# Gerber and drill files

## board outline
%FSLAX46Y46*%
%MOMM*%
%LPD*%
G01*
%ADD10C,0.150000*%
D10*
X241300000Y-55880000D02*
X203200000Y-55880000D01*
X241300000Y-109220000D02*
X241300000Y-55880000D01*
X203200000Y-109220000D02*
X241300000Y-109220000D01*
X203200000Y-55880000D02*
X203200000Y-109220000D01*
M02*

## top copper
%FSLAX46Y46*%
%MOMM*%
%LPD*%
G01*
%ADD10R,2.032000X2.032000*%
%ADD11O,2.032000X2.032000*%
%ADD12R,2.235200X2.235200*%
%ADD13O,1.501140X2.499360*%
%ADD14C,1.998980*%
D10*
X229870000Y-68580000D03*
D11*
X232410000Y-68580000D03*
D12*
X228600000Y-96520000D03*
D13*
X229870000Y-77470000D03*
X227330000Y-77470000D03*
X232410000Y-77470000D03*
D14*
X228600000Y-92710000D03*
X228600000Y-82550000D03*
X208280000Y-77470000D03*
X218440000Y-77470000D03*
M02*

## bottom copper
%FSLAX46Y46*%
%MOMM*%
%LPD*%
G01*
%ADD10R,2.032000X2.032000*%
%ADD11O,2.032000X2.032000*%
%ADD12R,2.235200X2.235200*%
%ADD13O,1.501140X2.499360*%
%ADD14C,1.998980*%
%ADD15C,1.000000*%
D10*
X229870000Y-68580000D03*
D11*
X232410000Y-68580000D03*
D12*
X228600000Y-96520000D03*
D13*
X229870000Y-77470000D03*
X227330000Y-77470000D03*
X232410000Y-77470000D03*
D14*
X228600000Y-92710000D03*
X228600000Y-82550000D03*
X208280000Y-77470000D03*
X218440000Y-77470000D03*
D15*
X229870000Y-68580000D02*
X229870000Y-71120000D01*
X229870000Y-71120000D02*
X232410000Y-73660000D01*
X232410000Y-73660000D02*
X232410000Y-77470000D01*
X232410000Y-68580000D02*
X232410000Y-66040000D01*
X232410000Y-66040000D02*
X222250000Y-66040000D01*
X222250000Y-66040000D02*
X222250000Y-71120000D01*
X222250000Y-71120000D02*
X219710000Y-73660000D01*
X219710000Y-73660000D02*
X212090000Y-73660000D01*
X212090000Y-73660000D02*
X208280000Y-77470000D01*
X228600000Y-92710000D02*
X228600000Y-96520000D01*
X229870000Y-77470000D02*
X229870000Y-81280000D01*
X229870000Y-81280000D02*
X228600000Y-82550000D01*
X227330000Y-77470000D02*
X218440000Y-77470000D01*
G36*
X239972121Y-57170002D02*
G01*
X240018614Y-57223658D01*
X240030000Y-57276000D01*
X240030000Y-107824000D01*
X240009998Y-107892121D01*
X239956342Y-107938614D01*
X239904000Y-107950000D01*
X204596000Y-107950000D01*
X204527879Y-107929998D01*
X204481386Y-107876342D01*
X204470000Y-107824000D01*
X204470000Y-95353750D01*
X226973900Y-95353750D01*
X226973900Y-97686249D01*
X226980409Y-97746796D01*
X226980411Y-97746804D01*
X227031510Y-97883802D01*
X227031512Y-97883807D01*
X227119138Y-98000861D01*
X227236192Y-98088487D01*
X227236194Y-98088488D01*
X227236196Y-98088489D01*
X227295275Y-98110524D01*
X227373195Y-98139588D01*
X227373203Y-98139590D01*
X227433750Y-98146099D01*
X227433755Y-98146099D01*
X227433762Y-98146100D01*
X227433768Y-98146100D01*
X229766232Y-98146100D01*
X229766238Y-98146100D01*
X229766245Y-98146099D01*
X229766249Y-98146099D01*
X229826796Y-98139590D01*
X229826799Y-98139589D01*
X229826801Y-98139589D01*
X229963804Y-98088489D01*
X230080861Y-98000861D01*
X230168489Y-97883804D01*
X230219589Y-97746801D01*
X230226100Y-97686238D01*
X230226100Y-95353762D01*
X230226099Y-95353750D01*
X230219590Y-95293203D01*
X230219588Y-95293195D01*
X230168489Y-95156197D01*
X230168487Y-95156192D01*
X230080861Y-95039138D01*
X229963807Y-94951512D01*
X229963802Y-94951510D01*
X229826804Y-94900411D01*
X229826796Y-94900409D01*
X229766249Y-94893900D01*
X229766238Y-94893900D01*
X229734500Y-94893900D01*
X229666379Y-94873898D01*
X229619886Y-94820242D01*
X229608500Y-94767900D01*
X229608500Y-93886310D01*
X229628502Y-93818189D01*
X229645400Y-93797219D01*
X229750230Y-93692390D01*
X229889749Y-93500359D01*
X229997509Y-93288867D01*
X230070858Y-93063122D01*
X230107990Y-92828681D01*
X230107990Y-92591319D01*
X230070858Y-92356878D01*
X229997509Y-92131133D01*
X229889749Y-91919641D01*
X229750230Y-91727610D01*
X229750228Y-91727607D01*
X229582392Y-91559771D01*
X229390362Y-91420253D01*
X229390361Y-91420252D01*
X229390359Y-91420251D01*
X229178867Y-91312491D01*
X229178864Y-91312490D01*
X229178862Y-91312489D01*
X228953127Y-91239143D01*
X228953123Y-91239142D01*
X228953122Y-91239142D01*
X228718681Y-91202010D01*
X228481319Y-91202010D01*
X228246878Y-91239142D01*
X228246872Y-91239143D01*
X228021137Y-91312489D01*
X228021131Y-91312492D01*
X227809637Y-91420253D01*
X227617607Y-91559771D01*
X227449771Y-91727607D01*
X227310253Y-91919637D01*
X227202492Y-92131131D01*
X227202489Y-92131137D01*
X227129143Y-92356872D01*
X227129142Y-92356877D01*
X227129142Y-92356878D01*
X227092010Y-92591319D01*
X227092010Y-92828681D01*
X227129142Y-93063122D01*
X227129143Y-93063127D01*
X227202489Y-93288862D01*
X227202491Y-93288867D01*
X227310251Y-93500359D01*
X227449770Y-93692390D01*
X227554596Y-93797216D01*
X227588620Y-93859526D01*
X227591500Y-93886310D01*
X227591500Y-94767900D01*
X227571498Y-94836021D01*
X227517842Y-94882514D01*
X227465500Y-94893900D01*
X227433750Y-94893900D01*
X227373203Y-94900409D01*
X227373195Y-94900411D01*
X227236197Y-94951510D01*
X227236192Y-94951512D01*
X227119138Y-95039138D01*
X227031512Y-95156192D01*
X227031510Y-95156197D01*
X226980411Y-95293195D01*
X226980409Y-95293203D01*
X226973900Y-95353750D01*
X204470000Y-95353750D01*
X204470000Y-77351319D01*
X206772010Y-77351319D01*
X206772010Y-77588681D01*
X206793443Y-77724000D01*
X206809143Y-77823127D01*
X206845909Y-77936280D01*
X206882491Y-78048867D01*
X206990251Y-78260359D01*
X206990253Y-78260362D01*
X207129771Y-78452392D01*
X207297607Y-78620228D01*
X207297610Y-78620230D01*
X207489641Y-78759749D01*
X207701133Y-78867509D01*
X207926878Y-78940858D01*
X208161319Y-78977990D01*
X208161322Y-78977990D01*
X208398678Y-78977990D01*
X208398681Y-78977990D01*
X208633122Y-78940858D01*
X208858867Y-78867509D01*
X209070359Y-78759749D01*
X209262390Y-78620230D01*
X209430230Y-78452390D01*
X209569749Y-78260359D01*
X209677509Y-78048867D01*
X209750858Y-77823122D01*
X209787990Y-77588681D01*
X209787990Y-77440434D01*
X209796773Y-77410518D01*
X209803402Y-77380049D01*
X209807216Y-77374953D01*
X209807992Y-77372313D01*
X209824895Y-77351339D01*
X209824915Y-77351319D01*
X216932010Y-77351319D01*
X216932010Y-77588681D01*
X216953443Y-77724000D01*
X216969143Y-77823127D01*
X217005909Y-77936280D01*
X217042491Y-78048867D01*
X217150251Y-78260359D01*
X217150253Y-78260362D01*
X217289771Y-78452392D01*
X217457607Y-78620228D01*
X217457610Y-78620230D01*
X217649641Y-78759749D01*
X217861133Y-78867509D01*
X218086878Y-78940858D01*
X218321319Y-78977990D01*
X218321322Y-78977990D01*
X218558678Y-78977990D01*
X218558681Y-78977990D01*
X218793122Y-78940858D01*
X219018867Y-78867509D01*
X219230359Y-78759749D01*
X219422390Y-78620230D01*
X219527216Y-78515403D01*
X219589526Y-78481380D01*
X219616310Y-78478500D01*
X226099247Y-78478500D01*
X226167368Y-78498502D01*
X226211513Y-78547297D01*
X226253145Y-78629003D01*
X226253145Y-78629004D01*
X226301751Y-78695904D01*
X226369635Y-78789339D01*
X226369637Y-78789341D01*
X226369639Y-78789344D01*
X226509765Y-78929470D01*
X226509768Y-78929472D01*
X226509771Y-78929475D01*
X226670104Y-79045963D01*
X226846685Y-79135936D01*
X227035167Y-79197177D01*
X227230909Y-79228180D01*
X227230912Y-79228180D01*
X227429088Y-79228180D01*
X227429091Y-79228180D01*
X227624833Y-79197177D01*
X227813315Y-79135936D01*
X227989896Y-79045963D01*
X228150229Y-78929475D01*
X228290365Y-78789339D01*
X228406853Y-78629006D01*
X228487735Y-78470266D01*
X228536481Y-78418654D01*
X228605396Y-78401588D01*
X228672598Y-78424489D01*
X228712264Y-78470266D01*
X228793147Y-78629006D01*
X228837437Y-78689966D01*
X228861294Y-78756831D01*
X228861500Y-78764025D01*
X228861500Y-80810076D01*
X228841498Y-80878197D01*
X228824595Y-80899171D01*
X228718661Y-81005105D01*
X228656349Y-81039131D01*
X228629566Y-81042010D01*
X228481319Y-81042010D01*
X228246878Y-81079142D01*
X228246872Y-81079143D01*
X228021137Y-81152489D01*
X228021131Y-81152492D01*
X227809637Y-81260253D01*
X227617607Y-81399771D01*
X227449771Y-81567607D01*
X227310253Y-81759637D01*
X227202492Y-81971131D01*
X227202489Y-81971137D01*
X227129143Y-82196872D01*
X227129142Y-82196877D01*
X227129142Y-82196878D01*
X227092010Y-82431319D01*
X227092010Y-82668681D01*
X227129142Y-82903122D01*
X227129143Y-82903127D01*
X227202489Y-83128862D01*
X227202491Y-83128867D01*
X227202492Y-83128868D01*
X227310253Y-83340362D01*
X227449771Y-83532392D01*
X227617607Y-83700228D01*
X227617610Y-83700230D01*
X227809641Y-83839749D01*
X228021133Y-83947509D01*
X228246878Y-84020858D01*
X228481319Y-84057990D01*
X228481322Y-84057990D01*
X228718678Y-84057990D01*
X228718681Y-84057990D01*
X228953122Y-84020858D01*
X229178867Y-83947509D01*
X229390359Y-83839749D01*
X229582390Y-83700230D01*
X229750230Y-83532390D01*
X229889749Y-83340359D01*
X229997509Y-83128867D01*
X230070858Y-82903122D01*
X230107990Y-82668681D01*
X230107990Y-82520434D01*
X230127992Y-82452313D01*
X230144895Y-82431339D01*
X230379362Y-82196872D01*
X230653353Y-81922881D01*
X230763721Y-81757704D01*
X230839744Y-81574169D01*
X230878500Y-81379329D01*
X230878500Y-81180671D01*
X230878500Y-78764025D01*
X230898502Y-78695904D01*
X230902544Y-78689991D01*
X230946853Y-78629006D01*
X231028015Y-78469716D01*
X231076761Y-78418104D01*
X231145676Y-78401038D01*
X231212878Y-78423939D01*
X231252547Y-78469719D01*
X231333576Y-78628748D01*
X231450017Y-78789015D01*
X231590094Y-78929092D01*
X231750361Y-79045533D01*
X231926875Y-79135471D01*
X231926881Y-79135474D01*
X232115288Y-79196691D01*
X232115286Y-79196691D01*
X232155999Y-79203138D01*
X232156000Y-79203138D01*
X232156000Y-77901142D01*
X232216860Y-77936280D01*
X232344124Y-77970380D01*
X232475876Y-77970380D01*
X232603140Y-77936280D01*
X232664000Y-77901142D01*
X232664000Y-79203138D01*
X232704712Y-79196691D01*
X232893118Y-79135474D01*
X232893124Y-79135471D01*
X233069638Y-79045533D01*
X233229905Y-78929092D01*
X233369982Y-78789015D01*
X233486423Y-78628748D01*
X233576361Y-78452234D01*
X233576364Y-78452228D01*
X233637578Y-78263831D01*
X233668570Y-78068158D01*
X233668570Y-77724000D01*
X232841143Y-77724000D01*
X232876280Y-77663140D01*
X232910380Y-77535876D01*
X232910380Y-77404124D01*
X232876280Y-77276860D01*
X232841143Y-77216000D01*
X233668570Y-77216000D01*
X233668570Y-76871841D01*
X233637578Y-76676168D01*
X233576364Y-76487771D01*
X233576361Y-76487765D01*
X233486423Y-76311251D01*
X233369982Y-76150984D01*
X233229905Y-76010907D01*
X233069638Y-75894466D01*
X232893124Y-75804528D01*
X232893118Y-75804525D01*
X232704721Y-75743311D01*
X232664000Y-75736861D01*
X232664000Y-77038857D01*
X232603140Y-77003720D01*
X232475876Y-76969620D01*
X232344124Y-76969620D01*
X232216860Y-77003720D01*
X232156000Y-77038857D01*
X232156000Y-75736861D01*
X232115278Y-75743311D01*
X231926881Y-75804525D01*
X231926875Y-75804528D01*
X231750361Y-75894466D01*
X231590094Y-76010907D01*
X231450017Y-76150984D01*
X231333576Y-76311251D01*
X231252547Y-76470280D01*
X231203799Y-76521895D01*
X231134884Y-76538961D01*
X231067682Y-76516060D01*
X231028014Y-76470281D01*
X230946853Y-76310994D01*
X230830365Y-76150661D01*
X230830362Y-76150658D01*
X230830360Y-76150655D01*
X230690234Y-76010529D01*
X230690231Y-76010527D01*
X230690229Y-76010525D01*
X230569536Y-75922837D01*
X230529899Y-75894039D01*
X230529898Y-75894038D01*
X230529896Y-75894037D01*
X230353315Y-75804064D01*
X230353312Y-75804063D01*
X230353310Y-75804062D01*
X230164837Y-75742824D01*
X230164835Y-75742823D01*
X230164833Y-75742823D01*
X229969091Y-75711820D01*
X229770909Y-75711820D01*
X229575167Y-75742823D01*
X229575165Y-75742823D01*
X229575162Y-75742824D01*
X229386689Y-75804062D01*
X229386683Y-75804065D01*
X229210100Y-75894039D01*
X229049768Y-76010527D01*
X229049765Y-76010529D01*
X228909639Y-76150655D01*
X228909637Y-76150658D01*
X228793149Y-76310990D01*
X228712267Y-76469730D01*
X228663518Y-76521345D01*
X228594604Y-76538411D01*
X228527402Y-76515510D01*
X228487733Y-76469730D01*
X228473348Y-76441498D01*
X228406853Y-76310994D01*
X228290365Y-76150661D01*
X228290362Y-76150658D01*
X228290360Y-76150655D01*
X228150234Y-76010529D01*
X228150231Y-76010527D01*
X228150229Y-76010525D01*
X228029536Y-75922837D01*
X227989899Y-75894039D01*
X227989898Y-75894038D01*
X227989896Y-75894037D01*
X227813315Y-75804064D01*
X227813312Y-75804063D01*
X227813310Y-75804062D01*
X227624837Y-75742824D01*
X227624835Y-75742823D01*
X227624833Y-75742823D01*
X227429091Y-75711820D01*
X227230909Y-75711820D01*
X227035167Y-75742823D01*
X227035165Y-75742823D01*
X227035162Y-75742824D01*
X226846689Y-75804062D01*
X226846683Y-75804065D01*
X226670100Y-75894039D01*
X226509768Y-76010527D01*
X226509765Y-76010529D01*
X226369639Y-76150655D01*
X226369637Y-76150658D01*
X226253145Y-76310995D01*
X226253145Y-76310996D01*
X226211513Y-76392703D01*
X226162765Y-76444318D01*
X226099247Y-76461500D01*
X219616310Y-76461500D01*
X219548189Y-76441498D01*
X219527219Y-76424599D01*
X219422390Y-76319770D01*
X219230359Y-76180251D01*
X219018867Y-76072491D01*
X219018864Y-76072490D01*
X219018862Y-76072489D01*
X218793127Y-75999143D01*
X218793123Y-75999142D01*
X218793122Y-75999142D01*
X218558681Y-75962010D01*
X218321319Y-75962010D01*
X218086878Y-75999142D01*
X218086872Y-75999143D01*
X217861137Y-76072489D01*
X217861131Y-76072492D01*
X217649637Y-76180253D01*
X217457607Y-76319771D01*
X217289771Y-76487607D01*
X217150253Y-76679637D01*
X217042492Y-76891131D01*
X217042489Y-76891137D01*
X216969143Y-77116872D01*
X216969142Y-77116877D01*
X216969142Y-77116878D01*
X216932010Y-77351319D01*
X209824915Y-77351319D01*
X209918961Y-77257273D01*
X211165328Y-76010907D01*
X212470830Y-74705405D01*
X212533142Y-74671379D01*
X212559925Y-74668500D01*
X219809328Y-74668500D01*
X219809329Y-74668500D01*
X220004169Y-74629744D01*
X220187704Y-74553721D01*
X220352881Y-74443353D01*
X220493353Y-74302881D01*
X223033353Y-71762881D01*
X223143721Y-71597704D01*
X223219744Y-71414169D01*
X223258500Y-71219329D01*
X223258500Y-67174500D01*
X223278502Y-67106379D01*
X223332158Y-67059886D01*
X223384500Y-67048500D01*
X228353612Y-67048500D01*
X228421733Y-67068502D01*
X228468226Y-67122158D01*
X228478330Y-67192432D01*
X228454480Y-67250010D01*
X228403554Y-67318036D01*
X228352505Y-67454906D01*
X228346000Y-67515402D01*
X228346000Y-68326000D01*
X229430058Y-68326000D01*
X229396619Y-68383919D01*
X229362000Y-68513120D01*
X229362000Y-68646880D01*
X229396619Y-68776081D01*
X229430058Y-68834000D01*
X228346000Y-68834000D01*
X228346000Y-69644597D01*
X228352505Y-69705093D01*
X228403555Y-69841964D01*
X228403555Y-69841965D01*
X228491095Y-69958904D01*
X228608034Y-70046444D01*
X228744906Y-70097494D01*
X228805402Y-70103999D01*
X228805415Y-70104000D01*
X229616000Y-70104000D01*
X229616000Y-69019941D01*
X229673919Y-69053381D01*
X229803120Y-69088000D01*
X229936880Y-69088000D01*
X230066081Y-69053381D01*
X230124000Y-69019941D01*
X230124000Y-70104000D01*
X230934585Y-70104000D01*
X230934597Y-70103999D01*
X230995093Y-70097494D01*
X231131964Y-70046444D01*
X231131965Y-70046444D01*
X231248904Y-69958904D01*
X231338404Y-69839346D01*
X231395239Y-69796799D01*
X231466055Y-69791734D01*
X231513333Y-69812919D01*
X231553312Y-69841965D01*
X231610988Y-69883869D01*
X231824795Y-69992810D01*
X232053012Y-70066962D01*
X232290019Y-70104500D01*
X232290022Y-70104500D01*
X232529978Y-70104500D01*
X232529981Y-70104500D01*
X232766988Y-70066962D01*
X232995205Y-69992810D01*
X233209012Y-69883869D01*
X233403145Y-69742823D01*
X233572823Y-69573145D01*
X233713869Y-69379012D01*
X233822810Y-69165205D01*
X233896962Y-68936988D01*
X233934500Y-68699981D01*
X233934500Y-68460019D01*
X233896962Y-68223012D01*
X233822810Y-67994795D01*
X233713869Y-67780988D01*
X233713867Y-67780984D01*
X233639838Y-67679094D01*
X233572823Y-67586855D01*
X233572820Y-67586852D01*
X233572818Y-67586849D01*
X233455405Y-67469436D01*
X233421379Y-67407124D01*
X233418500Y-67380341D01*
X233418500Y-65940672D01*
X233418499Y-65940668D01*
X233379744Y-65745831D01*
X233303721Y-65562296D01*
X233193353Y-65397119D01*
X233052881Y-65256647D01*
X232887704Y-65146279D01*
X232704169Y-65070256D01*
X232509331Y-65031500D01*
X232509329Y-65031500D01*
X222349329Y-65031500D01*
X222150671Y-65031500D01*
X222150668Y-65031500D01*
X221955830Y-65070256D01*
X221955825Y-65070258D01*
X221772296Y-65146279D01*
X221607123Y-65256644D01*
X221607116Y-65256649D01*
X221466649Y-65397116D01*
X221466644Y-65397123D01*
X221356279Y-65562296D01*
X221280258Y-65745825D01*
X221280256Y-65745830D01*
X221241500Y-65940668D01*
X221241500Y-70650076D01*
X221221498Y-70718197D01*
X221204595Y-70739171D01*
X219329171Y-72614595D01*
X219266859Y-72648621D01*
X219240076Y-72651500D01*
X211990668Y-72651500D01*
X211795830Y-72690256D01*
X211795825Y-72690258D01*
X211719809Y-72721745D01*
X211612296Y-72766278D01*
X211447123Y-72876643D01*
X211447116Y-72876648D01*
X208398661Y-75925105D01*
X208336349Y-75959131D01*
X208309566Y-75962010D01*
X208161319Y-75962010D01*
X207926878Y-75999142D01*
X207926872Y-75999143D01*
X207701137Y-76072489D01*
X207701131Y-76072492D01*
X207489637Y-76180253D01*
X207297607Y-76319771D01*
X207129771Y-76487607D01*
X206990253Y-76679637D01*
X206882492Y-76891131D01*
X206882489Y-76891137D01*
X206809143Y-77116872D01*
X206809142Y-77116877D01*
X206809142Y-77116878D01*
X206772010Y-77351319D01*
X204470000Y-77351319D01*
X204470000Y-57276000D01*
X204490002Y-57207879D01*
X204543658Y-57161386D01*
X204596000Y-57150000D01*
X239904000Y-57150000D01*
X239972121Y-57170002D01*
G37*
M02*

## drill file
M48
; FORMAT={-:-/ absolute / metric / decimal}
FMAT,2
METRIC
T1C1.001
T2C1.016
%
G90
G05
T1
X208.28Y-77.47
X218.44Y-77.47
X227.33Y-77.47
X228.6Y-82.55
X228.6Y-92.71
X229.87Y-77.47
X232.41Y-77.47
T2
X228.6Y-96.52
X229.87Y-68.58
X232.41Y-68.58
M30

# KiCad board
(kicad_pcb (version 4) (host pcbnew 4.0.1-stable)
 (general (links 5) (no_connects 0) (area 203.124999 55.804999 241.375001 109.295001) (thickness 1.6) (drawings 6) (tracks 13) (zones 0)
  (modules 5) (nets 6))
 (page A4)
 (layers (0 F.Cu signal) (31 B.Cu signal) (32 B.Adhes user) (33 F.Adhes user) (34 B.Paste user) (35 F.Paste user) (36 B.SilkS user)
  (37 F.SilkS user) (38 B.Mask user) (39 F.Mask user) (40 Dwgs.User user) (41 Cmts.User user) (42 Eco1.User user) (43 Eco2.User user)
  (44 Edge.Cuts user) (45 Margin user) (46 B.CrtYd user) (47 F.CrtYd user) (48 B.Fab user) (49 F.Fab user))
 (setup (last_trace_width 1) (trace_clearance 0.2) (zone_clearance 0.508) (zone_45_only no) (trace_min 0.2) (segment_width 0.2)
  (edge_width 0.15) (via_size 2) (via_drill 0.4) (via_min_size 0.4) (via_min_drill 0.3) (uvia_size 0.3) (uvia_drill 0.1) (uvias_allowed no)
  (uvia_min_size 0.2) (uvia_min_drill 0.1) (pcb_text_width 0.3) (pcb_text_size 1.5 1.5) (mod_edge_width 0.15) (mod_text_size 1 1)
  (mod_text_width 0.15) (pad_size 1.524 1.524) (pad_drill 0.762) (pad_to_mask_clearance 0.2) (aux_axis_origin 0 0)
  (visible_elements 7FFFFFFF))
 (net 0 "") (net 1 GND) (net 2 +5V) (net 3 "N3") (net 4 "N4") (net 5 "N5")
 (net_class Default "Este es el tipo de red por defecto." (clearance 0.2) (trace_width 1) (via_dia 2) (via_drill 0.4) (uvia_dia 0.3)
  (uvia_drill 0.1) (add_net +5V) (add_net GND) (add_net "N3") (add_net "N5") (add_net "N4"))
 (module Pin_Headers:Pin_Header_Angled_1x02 (layer F.Cu) (at 229.87 68.58 90) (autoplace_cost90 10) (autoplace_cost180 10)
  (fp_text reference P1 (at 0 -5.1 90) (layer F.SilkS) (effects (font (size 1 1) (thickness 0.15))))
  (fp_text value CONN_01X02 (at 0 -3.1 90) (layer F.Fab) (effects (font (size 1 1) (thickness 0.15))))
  (pad 1 thru_hole rect (at 0 0 90) (size 2.032 2.032) (drill 1.016) (layers *.Cu *.Mask F.SilkS) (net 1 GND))
  (pad 2 thru_hole oval (at 0 2.54 90) (size 2.032 2.032) (drill 1.016) (layers *.Cu *.Mask F.SilkS) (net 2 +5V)))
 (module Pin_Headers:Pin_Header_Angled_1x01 (layer F.Cu) (at 228.6 96.52 270)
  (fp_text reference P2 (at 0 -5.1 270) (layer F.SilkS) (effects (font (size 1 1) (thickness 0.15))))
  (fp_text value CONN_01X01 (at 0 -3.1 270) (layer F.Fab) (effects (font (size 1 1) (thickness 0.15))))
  (pad 1 thru_hole rect (at 0 0 270) (size 2.2352 2.2352) (drill 1.016) (layers *.Cu *.Mask F.SilkS) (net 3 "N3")))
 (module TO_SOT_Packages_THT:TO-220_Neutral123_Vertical (layer F.Cu) (at 229.87 77.47)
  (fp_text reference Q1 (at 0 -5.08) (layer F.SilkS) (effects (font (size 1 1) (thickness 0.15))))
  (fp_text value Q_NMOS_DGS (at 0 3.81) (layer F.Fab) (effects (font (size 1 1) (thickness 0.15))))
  (pad 2 thru_hole oval (at 0 0 90) (size 2.49936 1.50114) (drill 1.00076) (layers *.Cu *.Mask F.SilkS) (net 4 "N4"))
  (pad 1 thru_hole oval (at -2.54 0 90) (size 2.49936 1.50114) (drill 1.00076) (layers *.Cu *.Mask F.SilkS) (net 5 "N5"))
  (pad 3 thru_hole oval (at 2.54 0 90) (size 2.49936 1.50114) (drill 1.00076) (layers *.Cu *.Mask F.SilkS) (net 1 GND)))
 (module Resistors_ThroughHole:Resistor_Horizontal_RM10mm (layer F.Cu) (at 228.6 87.63 90)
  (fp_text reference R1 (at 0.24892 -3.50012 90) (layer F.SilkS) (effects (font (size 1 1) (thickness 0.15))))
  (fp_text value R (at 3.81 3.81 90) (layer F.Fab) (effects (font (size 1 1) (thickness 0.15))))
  (pad 1 thru_hole circle (at -5.08 0 90) (size 1.99898 1.99898) (drill 1.00076) (layers *.Cu *.SilkS *.Mask) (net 3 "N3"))
  (pad 2 thru_hole circle (at 5.08 0 90) (size 1.99898 1.99898) (drill 1.00076) (layers *.Cu *.SilkS *.Mask) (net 4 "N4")))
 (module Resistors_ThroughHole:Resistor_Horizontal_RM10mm (layer F.Cu) (at 213.36 77.47)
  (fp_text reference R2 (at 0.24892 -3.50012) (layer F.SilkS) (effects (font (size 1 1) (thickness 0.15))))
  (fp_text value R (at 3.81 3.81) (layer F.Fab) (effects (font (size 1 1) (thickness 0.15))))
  (pad 1 thru_hole circle (at -5.08 0) (size 1.99898 1.99898) (drill 1.00076) (layers *.Cu *.SilkS *.Mask) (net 2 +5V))
  (pad 2 thru_hole circle (at 5.08 0) (size 1.99898 1.99898) (drill 1.00076) (layers *.Cu *.SilkS *.Mask) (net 5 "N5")))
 (gr_line (start 241.3 55.88) (end 203.2 55.88) (angle 90) (layer Edge.Cuts) (width 0.15))
 (gr_line (start 241.3 109.22) (end 241.3 55.88) (angle 90) (layer Edge.Cuts) (width 0.15))
 (gr_line (start 203.2 109.22) (end 241.3 109.22) (angle 90) (layer Edge.Cuts) (width 0.15))
 (gr_line (start 203.2 55.88) (end 203.2 109.22) (angle 90) (layer Edge.Cuts) (width 0.15))
 (segment (start 229.87 68.58) (end 229.87 71.12) (width 1) (layer B.Cu) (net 1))
 (segment (start 229.87 71.12) (end 232.41 73.66) (width 1) (layer B.Cu) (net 1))
 (segment (start 232.41 73.66) (end 232.41 77.47) (width 1) (layer B.Cu) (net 1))
 (segment (start 232.41 68.58) (end 232.41 66.04) (width 1) (layer B.Cu) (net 2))
 (segment (start 232.41 66.04) (end 222.25 66.04) (width 1) (layer B.Cu) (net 2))
 (segment (start 222.25 66.04) (end 222.25 71.12) (width 1) (layer B.Cu) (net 2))
 (segment (start 222.25 71.12) (end 219.71 73.66) (width 1) (layer B.Cu) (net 2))
 (segment (start 219.71 73.66) (end 212.09 73.66) (width 1) (layer B.Cu) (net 2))
 (segment (start 212.09 73.66) (end 208.28 77.47) (width 1) (layer B.Cu) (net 2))
 (segment (start 228.6 92.71) (end 228.6 96.52) (width 1) (layer B.Cu) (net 3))
 (segment (start 229.87 77.47) (end 229.87 81.28) (width 1) (layer B.Cu) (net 4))
 (segment (start 229.87 81.28) (end 228.6 82.55) (width 1) (layer B.Cu) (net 4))
 (segment (start 227.33 77.47) (end 218.44 77.47) (width 1) (layer B.Cu) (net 5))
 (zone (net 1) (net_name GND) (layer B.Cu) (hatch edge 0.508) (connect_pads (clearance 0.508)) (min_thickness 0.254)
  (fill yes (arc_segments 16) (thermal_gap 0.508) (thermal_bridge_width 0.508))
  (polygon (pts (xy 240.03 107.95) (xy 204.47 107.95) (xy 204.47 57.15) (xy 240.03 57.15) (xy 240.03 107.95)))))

